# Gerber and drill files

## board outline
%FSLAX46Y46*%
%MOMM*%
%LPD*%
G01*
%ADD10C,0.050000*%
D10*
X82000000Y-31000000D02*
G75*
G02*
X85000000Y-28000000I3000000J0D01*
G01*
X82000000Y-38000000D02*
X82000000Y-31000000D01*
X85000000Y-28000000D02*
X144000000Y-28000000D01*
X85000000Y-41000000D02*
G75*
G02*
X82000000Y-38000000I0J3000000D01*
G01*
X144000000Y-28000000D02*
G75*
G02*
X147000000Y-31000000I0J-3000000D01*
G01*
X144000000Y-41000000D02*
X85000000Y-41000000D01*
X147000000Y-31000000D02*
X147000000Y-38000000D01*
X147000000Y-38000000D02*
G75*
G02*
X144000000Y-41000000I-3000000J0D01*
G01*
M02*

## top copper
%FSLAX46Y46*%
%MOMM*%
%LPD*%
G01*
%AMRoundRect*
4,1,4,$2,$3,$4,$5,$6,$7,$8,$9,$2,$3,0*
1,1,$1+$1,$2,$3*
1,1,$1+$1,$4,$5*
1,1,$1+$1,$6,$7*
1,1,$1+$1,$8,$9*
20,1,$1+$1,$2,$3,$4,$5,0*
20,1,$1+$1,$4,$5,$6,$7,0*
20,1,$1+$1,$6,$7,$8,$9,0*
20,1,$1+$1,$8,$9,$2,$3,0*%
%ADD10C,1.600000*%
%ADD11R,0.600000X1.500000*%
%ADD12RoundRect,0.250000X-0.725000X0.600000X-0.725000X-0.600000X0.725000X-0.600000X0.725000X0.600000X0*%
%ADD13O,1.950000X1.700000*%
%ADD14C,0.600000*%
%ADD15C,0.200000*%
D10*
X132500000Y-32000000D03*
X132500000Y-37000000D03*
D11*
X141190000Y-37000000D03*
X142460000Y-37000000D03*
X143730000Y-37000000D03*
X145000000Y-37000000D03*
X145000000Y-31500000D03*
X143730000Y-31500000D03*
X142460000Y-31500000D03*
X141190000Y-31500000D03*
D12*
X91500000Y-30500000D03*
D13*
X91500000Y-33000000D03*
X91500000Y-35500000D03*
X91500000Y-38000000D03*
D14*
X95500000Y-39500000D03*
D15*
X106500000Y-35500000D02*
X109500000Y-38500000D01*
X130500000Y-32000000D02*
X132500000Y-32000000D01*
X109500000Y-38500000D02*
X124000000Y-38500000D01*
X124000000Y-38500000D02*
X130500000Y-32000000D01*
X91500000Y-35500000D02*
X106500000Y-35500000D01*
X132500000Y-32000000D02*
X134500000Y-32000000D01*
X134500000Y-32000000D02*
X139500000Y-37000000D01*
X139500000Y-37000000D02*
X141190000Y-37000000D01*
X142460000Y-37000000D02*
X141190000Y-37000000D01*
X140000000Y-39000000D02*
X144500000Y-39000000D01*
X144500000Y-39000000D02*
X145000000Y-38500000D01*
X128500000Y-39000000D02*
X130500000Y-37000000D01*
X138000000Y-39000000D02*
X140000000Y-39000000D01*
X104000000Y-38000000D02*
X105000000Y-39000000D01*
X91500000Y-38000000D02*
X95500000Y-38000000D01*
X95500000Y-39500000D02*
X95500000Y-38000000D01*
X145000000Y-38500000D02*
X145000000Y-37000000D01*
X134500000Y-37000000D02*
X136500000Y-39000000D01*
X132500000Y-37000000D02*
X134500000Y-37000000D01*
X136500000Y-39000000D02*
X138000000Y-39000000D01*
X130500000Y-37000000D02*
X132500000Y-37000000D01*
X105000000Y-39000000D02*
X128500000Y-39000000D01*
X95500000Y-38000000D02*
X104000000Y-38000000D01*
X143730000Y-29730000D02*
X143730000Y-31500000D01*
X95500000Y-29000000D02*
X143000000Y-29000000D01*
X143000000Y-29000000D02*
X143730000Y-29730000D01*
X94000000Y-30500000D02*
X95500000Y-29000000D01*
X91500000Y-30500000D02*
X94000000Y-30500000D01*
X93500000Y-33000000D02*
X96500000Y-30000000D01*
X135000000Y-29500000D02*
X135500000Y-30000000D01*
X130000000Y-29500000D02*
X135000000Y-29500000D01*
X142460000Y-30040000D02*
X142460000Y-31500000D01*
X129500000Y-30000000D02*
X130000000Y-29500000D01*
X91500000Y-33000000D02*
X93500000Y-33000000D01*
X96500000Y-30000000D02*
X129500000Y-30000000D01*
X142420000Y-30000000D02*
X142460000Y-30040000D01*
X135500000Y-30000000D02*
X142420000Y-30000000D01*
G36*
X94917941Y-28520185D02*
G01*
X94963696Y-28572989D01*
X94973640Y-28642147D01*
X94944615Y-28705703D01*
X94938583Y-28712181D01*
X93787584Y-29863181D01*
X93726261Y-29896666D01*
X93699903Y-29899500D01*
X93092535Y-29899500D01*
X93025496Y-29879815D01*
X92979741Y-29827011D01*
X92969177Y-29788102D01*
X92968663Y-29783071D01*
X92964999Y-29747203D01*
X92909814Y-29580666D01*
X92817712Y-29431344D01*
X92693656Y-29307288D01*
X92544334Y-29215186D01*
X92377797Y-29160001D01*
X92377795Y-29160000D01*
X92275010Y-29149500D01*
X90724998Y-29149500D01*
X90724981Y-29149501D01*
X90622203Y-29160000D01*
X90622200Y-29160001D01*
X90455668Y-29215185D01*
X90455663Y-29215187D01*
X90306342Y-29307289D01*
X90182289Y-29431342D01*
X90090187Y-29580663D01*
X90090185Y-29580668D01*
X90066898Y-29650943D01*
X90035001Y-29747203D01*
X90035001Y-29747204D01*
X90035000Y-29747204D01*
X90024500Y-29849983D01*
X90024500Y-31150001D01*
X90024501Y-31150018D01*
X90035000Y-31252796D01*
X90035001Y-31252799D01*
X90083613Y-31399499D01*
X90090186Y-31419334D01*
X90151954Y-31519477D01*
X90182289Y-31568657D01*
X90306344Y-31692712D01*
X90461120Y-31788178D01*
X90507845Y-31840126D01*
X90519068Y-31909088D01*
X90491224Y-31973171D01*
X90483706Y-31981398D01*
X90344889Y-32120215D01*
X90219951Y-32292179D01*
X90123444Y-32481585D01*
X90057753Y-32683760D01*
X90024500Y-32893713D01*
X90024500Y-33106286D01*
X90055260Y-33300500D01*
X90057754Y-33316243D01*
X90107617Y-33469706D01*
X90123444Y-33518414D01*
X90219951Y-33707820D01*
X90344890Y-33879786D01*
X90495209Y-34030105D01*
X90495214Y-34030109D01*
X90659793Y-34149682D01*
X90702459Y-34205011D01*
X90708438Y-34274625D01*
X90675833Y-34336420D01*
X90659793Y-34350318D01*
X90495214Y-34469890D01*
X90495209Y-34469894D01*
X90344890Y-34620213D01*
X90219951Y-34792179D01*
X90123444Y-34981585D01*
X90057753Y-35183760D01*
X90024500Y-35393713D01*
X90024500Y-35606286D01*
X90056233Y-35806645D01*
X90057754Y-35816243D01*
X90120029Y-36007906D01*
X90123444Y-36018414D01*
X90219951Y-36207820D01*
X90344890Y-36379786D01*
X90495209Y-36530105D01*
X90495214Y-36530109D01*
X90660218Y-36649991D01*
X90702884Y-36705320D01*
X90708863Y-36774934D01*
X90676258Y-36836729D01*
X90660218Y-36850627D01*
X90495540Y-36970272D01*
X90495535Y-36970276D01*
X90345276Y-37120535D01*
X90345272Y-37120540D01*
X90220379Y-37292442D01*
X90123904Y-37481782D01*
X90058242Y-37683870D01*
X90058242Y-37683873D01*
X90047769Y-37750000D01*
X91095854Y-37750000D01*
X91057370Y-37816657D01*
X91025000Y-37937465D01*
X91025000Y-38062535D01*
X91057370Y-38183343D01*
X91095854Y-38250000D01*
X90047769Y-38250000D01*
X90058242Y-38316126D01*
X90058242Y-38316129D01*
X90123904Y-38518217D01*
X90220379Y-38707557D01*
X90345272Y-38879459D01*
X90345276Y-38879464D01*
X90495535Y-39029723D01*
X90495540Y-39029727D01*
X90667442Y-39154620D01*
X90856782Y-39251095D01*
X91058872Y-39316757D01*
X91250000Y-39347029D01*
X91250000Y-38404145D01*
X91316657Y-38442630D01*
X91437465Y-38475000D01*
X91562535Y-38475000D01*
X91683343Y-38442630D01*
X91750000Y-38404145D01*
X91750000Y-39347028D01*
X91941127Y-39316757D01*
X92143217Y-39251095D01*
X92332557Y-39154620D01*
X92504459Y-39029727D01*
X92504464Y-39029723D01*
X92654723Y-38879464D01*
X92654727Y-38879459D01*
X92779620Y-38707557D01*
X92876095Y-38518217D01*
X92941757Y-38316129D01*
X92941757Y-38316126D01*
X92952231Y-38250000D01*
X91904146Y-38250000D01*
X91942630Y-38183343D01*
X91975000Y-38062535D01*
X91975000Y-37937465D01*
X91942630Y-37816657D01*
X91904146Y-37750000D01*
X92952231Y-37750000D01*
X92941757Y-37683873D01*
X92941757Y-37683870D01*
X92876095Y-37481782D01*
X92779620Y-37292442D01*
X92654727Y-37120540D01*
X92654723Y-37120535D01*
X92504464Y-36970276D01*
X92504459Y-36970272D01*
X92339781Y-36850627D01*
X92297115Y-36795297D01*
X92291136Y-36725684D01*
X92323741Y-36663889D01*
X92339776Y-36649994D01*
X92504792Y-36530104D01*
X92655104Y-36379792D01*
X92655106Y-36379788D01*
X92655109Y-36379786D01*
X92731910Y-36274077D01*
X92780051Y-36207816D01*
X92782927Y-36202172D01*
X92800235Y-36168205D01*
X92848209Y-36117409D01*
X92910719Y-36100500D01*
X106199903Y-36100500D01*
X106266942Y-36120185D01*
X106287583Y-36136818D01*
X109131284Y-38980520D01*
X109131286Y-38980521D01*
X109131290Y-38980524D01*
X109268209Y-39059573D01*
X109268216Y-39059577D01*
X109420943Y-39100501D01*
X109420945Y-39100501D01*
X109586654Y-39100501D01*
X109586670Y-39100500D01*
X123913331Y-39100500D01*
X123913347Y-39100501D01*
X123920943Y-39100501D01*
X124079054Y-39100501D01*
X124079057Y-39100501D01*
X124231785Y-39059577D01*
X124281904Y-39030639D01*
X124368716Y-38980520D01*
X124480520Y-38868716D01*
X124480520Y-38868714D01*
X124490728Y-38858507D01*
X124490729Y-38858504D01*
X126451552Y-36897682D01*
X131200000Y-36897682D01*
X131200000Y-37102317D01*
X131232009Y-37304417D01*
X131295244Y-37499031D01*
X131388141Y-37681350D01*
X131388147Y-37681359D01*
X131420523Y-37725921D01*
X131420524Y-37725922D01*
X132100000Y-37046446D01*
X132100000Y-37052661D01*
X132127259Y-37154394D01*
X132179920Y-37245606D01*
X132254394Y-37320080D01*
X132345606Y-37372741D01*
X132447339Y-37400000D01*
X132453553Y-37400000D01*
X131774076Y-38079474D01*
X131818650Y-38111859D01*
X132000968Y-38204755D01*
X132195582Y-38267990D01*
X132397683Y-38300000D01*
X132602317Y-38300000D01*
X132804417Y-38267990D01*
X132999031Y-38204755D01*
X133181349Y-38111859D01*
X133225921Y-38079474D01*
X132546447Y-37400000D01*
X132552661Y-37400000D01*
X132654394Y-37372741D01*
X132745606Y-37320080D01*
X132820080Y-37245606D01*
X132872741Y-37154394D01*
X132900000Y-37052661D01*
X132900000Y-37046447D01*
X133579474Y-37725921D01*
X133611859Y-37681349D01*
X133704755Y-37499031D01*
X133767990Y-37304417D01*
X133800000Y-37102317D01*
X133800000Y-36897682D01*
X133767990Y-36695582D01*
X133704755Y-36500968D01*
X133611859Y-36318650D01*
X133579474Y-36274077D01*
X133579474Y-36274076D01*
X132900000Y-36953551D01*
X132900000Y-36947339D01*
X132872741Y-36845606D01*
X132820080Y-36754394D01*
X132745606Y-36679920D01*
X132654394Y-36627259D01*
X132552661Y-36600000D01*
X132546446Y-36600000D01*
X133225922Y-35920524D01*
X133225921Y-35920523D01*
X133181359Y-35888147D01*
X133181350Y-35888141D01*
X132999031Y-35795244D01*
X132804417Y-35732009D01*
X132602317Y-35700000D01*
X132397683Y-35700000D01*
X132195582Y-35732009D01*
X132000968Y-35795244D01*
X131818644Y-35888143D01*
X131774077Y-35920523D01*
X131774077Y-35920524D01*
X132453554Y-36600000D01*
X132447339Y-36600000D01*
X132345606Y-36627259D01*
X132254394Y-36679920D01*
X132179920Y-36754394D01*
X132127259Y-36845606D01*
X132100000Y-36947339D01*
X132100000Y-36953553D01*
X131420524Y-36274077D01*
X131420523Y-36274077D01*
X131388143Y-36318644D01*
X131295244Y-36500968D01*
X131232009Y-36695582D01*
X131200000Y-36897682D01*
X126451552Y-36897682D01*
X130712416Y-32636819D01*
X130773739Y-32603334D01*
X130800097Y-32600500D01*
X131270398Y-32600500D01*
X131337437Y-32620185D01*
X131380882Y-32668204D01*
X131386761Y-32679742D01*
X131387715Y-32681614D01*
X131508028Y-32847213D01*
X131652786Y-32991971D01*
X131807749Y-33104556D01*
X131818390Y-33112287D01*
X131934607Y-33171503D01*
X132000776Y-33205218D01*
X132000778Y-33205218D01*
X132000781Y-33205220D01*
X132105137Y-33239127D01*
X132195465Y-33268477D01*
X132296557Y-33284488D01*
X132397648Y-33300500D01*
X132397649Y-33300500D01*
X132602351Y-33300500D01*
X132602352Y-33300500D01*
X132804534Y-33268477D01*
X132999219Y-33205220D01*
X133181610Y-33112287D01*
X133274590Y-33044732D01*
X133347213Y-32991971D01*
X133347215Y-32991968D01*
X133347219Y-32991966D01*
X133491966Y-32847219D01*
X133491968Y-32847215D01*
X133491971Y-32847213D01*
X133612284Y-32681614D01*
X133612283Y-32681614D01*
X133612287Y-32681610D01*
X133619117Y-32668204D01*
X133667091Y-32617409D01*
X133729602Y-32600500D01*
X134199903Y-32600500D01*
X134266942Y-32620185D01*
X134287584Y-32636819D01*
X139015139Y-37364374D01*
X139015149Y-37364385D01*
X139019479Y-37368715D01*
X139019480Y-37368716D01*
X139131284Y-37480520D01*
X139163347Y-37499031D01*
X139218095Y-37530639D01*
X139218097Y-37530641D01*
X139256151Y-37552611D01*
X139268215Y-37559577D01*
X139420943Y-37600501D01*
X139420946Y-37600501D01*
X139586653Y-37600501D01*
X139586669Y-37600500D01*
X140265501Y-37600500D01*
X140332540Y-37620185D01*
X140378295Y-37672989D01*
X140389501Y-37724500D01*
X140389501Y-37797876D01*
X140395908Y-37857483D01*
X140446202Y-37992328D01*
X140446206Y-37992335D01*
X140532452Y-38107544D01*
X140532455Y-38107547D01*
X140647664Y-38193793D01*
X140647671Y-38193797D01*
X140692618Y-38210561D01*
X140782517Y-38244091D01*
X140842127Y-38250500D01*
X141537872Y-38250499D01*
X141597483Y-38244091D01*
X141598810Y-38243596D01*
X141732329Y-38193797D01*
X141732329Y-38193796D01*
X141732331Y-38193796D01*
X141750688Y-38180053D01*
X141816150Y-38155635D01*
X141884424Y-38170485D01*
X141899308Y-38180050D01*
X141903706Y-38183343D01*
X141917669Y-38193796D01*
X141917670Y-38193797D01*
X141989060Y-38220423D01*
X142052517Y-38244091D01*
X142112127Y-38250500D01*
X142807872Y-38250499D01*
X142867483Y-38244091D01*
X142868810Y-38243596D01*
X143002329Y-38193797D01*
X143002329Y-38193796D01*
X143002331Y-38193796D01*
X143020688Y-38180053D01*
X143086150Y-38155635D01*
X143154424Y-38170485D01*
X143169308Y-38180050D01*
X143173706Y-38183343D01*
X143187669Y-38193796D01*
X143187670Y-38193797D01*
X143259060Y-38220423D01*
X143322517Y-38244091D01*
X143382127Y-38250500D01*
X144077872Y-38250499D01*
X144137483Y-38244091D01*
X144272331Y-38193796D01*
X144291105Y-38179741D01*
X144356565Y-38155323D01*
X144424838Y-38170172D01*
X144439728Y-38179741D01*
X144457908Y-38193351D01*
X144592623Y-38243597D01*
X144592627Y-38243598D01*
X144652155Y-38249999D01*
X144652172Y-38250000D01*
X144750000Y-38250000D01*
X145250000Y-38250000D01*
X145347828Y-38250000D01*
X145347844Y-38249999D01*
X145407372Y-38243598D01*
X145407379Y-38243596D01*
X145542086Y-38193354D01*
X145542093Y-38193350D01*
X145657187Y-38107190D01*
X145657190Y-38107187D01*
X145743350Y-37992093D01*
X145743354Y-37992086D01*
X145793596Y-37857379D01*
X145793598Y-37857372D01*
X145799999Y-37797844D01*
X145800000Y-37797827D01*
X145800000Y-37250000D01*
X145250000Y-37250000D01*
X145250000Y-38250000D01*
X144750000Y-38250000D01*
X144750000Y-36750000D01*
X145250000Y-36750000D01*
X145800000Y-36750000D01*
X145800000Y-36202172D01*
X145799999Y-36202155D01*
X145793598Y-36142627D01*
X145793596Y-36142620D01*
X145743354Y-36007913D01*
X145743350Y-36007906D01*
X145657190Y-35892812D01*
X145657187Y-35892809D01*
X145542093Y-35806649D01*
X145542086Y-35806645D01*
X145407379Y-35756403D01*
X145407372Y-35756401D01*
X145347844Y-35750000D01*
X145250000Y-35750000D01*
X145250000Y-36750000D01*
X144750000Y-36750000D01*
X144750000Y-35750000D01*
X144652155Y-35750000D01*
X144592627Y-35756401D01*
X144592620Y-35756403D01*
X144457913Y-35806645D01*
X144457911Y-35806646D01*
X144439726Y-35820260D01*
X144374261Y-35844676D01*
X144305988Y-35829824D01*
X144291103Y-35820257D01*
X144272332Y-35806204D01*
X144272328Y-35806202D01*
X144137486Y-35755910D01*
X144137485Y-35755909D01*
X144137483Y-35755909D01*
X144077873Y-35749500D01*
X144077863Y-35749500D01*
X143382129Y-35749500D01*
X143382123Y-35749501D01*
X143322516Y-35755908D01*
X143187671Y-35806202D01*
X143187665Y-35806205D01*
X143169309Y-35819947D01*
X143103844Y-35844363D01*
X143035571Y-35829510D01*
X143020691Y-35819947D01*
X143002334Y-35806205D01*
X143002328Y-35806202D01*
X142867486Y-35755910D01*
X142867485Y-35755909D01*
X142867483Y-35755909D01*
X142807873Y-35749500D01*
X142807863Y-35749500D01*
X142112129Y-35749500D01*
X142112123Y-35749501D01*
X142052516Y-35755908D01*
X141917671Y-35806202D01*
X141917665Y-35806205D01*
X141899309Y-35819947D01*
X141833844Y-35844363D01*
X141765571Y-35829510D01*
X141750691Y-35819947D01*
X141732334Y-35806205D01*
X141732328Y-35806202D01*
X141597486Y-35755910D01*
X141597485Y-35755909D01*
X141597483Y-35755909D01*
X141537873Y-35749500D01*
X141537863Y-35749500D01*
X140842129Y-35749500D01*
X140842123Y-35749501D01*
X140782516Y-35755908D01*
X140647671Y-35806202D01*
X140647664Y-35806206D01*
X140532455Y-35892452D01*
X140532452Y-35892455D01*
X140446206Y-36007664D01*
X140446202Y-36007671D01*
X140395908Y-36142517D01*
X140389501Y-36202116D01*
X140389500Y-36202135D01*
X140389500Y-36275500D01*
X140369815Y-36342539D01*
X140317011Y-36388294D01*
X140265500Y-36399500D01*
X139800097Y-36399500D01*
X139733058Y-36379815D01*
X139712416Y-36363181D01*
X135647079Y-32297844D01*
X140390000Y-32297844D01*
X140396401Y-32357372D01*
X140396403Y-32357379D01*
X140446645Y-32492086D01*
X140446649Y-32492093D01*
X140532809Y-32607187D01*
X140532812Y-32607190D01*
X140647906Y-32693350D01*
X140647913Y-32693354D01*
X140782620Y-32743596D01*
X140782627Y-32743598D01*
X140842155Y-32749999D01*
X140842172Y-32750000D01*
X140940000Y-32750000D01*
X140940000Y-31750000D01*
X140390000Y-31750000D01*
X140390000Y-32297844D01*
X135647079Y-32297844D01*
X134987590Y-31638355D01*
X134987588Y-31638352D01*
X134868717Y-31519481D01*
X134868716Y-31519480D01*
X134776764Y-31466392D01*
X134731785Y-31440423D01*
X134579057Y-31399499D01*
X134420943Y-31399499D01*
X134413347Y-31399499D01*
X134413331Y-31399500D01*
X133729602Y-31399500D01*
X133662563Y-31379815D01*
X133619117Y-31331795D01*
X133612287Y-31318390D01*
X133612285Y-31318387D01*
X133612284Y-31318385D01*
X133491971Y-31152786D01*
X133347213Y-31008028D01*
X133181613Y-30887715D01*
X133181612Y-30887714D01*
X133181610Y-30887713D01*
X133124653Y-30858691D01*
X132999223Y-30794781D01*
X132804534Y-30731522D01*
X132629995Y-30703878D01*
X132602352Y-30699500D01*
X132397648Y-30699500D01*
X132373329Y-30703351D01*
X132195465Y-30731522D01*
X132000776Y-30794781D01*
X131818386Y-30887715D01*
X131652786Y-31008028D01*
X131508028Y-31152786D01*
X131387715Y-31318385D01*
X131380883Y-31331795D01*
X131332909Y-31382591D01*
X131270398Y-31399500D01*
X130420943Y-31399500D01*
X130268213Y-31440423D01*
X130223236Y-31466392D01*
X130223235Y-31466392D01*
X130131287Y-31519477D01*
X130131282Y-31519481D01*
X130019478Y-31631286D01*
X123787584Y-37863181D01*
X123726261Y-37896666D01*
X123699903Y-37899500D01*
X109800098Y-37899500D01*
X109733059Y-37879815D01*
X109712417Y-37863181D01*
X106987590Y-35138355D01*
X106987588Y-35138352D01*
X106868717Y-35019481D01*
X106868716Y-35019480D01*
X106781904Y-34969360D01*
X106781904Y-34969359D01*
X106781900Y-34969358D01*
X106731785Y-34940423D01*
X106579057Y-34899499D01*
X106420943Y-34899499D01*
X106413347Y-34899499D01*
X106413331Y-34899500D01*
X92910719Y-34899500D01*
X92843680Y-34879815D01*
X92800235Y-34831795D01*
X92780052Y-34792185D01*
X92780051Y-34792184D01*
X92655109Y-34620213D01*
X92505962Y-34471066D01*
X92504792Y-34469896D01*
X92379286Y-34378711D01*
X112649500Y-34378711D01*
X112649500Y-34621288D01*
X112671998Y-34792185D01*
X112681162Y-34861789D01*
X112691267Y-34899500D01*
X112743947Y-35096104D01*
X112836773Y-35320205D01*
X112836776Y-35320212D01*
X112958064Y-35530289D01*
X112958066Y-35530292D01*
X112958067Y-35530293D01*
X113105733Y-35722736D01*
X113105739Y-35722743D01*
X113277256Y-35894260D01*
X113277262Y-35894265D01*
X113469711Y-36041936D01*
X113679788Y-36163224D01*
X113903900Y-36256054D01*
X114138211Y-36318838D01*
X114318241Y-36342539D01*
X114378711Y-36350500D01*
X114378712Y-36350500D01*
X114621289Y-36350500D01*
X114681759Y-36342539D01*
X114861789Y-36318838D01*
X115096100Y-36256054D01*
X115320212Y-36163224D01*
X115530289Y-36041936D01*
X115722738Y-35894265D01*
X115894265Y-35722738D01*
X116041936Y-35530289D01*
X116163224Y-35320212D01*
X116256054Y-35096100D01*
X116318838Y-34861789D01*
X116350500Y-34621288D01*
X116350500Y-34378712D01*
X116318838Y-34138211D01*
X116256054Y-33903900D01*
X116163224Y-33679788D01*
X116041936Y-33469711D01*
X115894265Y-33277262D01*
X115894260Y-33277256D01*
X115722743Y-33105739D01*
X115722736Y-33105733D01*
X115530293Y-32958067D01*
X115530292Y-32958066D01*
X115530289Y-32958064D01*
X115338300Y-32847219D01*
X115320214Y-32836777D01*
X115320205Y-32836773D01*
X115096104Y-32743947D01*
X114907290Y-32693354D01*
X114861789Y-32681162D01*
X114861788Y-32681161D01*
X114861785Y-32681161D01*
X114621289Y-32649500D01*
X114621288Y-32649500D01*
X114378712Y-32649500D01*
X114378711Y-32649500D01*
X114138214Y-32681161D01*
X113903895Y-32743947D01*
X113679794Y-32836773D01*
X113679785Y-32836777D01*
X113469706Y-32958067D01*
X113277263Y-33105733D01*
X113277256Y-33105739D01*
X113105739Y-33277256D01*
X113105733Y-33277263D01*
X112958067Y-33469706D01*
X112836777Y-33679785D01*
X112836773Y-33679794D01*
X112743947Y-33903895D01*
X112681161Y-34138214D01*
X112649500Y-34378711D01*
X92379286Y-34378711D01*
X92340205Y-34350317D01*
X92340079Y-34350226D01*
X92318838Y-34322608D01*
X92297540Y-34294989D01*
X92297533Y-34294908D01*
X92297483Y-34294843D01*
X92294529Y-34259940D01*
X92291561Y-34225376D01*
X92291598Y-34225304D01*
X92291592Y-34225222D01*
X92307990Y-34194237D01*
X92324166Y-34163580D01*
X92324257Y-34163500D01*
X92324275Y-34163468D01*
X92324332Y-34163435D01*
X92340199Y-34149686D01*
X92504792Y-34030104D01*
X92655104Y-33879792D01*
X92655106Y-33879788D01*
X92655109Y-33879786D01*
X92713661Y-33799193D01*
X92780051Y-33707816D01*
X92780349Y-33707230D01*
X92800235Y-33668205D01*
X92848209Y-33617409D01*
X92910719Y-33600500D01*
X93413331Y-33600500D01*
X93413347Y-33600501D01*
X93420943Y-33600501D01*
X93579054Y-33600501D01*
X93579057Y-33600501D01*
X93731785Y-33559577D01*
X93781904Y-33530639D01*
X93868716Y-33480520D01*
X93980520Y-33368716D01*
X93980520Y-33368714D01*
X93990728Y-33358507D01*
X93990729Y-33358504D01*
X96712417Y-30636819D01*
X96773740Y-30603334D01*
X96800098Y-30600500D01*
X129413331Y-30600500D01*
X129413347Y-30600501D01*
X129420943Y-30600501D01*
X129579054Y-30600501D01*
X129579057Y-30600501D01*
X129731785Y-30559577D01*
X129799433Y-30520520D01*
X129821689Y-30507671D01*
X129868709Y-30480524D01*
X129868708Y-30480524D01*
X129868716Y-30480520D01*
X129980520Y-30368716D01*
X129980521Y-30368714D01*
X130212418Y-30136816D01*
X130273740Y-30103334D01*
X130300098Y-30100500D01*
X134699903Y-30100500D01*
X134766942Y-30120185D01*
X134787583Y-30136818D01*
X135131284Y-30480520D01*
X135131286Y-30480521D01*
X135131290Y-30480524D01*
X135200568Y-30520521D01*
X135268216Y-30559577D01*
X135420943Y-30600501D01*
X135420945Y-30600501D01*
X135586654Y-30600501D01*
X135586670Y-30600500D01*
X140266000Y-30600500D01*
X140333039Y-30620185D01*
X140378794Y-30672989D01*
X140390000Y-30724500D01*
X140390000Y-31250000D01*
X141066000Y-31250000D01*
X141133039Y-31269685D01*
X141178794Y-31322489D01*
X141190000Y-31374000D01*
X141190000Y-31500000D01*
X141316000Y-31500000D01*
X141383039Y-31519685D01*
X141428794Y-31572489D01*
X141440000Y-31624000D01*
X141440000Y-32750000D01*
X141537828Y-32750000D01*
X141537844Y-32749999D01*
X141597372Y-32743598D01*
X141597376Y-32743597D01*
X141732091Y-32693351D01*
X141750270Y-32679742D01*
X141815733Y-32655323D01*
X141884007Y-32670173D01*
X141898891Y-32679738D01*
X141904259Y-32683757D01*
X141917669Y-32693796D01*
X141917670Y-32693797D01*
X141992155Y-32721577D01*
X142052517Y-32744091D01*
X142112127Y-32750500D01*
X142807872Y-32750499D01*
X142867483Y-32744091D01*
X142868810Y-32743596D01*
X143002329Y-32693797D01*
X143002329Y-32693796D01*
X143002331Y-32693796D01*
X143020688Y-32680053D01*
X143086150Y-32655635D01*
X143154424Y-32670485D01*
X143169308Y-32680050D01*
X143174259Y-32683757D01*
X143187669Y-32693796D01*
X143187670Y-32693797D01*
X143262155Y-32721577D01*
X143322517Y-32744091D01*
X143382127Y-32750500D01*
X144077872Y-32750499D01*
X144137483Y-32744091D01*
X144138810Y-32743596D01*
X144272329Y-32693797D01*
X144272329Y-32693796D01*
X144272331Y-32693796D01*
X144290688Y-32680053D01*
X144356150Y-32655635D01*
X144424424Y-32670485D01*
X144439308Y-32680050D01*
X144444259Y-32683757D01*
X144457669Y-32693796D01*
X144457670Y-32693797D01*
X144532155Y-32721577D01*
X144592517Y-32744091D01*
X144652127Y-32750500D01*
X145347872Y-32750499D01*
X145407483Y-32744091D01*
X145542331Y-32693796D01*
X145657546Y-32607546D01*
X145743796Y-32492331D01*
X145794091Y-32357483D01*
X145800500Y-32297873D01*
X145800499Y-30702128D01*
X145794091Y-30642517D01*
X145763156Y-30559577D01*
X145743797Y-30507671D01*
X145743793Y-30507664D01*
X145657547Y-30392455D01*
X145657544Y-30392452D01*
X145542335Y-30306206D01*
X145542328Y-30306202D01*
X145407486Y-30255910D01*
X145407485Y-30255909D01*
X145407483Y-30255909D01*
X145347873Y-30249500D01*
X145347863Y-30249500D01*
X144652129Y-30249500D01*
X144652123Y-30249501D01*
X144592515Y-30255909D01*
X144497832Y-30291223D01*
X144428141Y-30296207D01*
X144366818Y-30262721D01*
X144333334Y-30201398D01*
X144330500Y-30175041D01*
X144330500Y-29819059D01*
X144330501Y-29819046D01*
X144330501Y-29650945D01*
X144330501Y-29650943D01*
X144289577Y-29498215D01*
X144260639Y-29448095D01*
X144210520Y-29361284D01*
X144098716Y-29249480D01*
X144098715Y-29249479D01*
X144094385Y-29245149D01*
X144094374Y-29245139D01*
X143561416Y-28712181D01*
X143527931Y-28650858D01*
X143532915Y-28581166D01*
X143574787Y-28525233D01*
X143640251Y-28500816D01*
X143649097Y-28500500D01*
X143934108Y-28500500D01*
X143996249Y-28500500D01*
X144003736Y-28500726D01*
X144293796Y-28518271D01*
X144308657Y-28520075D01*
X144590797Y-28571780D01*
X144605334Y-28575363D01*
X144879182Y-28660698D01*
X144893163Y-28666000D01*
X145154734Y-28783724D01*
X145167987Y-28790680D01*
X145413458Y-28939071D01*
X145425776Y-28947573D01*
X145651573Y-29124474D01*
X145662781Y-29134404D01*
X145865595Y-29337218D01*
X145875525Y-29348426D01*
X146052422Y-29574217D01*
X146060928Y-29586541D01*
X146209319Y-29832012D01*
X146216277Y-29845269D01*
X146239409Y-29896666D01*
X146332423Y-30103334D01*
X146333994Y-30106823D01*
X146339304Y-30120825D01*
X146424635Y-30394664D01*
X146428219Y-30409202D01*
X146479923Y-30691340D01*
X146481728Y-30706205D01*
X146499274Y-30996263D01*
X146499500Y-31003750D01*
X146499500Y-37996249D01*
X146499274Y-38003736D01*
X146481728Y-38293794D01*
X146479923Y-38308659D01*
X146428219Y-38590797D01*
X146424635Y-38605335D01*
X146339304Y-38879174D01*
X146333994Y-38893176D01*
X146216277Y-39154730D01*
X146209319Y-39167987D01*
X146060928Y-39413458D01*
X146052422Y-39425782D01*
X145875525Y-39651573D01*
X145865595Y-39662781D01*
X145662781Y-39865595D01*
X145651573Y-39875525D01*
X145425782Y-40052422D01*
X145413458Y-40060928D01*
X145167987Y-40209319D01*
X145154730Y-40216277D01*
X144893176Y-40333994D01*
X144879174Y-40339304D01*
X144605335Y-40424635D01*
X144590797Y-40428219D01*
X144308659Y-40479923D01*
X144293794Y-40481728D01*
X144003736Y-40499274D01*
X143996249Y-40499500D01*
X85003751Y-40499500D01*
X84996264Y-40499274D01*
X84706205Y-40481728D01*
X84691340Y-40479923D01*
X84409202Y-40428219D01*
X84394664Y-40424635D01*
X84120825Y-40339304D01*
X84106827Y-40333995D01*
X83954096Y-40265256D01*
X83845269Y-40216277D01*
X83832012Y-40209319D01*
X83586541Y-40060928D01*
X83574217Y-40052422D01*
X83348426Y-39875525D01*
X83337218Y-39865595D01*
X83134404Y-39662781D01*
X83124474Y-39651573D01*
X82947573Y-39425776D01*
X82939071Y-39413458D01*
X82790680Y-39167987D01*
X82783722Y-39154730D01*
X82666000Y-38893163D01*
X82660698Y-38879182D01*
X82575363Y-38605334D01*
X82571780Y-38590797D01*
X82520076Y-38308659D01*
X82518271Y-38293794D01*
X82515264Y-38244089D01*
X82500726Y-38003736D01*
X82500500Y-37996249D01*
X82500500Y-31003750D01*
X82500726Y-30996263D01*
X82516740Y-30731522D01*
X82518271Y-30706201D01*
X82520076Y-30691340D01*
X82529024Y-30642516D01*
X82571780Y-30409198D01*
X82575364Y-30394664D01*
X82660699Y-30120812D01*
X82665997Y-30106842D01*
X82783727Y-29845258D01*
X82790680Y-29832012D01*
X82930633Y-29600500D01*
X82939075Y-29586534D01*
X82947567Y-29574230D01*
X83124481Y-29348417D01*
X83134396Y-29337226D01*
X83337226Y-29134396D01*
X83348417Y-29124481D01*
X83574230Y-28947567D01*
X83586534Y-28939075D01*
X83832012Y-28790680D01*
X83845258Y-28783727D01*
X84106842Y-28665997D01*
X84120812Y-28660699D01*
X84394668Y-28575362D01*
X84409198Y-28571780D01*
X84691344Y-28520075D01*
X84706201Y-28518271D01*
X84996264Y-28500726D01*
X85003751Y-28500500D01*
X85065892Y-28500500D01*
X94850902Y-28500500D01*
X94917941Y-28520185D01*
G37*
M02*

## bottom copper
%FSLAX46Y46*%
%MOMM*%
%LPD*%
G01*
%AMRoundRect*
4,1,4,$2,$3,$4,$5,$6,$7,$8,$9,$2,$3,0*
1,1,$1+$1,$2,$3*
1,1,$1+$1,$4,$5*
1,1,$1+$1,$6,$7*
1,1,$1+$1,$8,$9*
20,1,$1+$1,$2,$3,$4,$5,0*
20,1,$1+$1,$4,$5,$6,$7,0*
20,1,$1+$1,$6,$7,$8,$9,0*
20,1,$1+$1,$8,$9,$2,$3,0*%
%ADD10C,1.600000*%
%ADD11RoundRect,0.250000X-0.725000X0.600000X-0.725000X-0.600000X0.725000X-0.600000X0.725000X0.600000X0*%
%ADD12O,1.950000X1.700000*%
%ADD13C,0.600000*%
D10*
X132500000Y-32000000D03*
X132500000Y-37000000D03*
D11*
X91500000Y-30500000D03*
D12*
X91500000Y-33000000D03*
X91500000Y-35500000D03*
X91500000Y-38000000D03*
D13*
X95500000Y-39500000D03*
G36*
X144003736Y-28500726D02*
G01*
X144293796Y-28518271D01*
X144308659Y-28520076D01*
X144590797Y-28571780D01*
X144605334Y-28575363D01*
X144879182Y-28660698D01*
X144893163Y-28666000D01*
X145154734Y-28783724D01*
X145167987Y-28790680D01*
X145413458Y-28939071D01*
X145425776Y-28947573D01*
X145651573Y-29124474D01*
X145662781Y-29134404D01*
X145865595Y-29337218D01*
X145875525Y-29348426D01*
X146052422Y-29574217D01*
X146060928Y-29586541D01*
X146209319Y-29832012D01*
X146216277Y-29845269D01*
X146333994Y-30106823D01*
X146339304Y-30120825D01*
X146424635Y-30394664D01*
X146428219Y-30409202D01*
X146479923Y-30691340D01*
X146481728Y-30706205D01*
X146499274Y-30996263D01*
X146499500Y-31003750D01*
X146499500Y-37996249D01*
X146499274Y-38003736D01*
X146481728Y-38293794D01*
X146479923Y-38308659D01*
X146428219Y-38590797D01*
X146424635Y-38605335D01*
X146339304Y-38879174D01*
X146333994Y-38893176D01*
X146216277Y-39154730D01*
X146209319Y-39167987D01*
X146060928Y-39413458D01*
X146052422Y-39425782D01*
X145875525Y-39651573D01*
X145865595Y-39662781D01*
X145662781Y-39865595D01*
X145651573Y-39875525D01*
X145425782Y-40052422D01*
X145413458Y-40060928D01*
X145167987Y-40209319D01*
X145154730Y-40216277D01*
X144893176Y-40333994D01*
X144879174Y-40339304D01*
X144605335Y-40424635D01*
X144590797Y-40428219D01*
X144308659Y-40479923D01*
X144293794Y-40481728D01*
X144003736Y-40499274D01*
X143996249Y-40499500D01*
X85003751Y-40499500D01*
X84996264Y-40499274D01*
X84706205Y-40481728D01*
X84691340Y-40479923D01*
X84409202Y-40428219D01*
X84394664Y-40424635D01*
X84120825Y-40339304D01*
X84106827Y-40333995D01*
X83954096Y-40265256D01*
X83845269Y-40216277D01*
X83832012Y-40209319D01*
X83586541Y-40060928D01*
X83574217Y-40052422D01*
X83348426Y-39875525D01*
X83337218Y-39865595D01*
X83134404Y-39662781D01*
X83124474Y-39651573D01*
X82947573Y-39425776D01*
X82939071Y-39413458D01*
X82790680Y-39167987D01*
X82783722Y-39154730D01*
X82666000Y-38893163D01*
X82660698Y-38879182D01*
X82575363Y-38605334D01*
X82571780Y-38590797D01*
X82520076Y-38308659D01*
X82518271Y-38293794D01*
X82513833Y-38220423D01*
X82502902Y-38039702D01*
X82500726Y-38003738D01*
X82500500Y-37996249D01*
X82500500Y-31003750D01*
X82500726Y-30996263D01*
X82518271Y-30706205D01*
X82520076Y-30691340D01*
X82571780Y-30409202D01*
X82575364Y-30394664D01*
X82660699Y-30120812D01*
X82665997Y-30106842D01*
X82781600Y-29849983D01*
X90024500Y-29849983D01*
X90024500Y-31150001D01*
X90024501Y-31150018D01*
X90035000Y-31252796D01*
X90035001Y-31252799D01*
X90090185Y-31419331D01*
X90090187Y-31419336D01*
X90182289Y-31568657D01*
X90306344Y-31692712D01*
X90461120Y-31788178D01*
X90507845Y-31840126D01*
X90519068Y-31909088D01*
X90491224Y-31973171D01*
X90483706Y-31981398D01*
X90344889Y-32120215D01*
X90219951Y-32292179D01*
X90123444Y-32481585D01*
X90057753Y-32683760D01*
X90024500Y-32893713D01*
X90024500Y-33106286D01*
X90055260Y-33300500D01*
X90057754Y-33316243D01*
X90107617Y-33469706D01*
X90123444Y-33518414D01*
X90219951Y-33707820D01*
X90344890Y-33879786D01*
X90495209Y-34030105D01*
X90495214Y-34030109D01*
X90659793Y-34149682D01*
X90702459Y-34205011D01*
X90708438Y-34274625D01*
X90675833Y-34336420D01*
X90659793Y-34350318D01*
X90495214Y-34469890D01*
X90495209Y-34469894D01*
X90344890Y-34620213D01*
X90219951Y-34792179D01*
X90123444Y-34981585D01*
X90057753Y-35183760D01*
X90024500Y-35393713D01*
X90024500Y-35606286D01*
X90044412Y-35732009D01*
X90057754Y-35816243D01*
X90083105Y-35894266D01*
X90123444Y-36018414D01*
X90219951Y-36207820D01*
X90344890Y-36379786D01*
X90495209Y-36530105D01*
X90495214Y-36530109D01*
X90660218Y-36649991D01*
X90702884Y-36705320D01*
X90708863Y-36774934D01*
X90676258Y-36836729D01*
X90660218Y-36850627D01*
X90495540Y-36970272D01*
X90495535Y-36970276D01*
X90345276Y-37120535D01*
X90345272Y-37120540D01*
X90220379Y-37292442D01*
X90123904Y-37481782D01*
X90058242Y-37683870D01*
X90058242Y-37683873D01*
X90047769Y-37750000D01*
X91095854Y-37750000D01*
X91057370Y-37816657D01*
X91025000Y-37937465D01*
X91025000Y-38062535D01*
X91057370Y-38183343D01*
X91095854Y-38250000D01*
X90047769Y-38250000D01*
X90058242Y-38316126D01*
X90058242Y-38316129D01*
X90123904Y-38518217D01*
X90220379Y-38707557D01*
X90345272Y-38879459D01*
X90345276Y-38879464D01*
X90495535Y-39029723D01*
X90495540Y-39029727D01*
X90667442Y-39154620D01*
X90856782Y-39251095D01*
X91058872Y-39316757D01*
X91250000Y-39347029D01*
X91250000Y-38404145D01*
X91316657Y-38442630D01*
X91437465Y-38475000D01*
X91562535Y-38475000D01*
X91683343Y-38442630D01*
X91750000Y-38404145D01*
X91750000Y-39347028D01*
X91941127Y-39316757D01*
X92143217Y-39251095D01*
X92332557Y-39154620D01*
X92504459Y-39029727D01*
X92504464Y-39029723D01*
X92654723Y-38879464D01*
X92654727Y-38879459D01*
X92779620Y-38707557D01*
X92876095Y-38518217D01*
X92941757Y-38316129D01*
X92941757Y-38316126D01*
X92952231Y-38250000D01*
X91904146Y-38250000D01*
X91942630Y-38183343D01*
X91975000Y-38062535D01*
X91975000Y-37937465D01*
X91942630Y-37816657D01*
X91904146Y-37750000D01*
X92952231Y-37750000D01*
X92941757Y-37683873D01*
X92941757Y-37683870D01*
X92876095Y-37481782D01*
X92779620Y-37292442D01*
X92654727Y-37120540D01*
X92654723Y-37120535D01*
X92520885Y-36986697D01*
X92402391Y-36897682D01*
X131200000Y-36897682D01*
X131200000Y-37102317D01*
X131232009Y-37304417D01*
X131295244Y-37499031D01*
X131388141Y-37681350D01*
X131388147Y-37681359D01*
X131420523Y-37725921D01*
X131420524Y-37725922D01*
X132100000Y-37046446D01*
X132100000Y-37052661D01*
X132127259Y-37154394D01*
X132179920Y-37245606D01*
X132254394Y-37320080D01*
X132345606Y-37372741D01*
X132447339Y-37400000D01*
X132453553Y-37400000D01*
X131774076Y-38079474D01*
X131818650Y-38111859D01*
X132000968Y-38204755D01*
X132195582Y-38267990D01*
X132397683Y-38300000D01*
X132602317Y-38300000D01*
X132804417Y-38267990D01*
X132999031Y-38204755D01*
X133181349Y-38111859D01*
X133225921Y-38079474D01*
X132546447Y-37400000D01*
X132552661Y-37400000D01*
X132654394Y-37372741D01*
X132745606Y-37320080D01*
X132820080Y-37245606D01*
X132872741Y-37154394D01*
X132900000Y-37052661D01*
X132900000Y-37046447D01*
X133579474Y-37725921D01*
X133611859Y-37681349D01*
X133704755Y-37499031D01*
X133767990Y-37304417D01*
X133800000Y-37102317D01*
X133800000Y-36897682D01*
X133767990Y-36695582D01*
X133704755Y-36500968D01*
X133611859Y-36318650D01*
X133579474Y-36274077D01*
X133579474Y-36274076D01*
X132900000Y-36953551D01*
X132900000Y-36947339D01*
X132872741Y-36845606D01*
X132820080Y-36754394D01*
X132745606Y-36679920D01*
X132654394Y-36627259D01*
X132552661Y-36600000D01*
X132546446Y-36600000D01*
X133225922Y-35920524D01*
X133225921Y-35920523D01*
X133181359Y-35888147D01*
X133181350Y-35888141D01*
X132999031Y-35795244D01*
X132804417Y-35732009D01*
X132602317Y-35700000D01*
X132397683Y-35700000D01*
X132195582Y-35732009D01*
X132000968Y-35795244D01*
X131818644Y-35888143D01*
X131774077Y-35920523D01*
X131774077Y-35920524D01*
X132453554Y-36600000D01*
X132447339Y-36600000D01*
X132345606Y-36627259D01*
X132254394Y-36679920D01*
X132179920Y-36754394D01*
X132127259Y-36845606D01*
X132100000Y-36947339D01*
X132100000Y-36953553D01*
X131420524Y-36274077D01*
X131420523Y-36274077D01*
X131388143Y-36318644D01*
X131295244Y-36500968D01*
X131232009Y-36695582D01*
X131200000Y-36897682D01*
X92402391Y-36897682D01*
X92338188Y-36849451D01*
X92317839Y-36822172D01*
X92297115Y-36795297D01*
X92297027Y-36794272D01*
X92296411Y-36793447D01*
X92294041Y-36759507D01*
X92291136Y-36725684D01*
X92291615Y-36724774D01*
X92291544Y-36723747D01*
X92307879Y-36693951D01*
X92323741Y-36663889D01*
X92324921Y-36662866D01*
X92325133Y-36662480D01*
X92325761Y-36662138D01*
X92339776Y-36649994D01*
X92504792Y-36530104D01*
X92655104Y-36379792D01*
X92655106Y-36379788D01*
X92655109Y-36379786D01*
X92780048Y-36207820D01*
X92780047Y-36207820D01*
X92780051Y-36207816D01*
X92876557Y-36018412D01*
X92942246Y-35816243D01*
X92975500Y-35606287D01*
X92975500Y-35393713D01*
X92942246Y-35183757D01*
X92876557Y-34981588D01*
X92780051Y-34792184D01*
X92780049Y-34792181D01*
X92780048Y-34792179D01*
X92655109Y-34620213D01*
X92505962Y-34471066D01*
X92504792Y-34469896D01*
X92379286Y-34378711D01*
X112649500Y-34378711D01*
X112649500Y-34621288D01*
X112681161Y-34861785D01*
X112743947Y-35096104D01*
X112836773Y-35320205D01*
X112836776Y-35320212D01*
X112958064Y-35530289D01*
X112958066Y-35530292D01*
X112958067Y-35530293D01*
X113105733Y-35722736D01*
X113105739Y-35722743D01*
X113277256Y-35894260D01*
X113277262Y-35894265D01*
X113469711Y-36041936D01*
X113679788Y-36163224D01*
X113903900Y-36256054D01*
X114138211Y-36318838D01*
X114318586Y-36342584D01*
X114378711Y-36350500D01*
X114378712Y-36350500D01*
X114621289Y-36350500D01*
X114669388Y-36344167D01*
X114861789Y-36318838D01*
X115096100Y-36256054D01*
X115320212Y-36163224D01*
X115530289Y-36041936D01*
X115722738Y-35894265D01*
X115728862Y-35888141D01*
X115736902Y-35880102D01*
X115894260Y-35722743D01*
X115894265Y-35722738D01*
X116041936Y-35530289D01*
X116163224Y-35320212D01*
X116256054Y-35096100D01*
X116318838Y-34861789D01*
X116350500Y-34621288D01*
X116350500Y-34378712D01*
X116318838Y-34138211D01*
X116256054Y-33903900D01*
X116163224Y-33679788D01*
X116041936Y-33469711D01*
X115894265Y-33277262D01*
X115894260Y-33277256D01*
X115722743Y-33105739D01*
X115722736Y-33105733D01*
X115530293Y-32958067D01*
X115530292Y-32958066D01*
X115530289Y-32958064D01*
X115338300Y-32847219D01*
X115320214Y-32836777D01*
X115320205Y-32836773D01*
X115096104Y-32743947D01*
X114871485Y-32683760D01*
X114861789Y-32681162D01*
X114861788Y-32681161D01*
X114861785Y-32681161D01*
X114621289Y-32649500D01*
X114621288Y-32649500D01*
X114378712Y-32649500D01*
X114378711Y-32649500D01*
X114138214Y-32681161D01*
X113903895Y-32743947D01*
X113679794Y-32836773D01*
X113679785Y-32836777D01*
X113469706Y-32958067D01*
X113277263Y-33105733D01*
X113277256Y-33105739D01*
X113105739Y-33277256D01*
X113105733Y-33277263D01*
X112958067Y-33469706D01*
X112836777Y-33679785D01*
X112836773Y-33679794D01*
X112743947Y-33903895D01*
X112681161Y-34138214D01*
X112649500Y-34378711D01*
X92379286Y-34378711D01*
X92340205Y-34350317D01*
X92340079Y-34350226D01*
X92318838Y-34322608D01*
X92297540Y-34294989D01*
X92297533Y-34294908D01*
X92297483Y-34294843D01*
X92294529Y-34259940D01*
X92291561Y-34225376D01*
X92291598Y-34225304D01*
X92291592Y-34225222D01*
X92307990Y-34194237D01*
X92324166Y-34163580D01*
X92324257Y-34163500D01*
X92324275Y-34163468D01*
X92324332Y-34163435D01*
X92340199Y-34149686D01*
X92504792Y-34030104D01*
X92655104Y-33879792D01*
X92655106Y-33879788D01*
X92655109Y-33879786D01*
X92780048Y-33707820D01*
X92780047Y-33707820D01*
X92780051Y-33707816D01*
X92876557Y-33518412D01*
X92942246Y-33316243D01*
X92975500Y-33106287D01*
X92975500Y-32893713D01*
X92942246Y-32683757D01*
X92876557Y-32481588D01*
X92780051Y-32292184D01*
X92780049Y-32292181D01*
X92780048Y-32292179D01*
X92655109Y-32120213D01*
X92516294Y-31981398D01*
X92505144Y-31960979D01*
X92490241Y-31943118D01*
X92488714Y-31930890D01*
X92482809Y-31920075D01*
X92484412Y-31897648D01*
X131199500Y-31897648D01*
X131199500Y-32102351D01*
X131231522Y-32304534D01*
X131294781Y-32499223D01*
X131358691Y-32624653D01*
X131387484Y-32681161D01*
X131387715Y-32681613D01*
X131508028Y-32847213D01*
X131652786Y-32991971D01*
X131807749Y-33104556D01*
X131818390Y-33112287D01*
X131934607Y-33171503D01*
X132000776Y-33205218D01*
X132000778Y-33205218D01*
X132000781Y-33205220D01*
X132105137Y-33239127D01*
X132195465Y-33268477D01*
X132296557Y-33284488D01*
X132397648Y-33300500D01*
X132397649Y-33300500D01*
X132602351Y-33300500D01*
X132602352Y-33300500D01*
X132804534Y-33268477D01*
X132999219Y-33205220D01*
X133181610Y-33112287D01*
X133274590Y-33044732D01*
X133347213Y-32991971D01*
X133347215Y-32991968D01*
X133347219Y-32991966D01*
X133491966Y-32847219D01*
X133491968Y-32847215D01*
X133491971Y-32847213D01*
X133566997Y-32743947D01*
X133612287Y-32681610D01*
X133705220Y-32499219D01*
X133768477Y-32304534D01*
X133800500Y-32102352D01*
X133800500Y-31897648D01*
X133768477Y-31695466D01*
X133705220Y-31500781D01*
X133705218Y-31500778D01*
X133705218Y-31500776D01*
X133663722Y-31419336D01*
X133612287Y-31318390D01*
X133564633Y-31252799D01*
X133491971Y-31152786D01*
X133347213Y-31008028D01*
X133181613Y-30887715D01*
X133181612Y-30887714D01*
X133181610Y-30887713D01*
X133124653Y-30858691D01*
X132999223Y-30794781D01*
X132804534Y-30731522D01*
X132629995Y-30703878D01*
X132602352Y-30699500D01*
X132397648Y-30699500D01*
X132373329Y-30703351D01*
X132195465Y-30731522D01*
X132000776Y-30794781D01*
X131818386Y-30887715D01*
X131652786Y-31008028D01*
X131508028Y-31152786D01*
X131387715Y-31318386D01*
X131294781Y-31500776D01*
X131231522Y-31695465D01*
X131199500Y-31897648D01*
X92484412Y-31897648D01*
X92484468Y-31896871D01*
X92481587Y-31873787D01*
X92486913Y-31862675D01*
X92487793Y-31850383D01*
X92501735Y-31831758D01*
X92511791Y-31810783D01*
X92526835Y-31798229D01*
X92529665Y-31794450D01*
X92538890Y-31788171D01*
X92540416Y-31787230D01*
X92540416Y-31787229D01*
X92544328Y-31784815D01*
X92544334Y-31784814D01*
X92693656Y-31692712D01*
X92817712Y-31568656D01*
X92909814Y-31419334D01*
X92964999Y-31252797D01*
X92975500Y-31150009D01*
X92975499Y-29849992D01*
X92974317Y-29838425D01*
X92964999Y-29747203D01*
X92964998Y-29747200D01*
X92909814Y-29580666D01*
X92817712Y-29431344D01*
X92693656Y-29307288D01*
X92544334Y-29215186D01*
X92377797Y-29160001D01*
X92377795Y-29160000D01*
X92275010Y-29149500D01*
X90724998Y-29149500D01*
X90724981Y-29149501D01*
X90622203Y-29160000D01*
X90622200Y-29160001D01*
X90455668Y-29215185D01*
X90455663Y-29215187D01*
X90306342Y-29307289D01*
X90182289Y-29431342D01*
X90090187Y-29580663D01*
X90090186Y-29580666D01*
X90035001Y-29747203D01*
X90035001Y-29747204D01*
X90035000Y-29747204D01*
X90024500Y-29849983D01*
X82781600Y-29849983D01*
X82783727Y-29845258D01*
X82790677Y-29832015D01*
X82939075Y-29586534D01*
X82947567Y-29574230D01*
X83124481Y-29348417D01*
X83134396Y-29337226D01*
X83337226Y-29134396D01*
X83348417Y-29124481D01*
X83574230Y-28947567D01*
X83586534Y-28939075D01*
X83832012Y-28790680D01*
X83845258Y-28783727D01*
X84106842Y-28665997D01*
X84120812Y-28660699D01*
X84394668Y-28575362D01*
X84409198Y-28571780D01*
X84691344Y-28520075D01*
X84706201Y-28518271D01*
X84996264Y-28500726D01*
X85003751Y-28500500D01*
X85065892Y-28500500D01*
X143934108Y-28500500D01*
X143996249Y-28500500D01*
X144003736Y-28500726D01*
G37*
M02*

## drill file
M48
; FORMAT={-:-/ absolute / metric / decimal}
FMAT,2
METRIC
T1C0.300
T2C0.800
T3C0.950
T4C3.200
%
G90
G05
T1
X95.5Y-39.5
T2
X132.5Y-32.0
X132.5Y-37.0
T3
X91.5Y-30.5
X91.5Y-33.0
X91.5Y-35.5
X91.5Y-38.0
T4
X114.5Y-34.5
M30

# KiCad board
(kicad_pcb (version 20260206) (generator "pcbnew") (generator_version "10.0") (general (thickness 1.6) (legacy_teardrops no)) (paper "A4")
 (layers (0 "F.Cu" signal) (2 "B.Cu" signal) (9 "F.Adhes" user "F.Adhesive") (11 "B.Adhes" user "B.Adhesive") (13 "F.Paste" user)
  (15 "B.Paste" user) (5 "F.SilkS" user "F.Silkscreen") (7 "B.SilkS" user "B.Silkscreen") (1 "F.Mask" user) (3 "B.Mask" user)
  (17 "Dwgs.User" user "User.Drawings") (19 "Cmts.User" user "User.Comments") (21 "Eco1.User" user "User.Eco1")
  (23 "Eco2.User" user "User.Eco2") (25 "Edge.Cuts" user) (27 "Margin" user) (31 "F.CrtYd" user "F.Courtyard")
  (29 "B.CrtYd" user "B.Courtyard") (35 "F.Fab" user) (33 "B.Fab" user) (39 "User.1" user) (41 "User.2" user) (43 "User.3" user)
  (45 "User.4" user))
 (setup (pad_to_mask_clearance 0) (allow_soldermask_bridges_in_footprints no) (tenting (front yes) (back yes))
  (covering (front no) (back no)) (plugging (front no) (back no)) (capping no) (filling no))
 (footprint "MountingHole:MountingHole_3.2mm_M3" (layer "F.Cu") (at 114.5 34.5)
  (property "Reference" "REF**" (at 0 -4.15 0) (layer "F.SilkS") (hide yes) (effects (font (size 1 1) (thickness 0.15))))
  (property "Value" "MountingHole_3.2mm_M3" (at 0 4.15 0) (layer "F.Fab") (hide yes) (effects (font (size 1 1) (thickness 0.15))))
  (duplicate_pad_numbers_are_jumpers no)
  (pad "" np_thru_hole circle (at 0 0) (size 3.2 3.2) (drill 3.2) (layers "*.Cu" "*.Mask")))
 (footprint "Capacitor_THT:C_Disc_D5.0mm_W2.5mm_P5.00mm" (layer "F.Cu") (at 132.5 32 -90)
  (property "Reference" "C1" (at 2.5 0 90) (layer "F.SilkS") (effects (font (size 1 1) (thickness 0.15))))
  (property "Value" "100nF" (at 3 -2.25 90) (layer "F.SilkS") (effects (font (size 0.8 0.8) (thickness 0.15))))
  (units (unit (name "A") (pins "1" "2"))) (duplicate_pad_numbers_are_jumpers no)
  (pad "1" thru_hole circle (at 0 0 270) (size 1.6 1.6) (drill 0.8) (layers "*.Cu" "*.Mask") (remove_unused_layers no)
   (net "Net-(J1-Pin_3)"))
  (pad "2" thru_hole circle (at 5 0 270) (size 1.6 1.6) (drill 0.8) (layers "*.Cu" "*.Mask") (remove_unused_layers no)
   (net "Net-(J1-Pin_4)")))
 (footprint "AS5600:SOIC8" (layer "F.Cu") (at 143.095 34.25)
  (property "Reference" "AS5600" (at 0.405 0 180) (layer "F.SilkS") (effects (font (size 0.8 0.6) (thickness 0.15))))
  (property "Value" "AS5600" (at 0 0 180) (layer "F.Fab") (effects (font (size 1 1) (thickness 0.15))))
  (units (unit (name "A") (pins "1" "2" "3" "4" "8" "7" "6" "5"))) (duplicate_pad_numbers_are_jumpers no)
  (pad "1" smd rect (at -1.905 2.75) (size 0.6 1.5) (layers "F.Cu" "F.Mask" "F.Paste") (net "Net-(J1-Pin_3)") (solder_mask_margin 0.102))
  (pad "2" smd rect (at -0.635 2.75) (size 0.6 1.5) (layers "F.Cu" "F.Mask" "F.Paste") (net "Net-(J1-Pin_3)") (solder_mask_margin 0.102))
  (pad "3" smd rect (at 0.635 2.75) (size 0.6 1.5) (layers "F.Cu" "F.Mask" "F.Paste") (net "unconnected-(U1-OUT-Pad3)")
   (solder_mask_margin 0.102))
  (pad "4" smd rect (at 1.905 2.75) (size 0.6 1.5) (layers "F.Cu" "F.Mask" "F.Paste") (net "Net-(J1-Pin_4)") (solder_mask_margin 0.102))
  (pad "5" smd rect (at 1.905 -2.75) (size 0.6 1.5) (layers "F.Cu" "F.Mask" "F.Paste") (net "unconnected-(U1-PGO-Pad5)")
   (solder_mask_margin 0.102))
  (pad "6" smd rect (at 0.635 -2.75) (size 0.6 1.5) (layers "F.Cu" "F.Mask" "F.Paste") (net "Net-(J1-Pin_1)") (solder_mask_margin 0.102))
  (pad "7" smd rect (at -0.635 -2.75) (size 0.6 1.5) (layers "F.Cu" "F.Mask" "F.Paste") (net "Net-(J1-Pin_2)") (solder_mask_margin 0.102))
  (pad "8" smd rect (at -1.905 -2.75) (size 0.6 1.5) (layers "F.Cu" "F.Mask" "F.Paste") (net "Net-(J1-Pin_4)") (solder_mask_margin 0.102)))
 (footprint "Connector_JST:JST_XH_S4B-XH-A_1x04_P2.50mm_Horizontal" (layer "F.Cu") (at 91.5 30.5 -90)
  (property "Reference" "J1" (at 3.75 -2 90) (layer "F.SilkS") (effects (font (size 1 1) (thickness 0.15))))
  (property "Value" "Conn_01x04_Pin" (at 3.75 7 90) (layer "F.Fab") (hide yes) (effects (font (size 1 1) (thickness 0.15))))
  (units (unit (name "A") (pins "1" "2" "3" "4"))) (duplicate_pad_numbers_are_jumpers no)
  (pad "1" thru_hole roundrect (at 0 0 270) (size 1.7 1.95) (drill 0.95) (layers "*.Cu" "*.Mask") (remove_unused_layers no)
   (roundrect_rratio 0.147059) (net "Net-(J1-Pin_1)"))
  (pad "2" thru_hole oval (at 2.5 0 270) (size 1.7 1.95) (drill 0.95) (layers "*.Cu" "*.Mask") (remove_unused_layers no)
   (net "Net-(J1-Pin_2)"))
  (pad "3" thru_hole oval (at 5 0 270) (size 1.7 1.95) (drill 0.95) (layers "*.Cu" "*.Mask") (remove_unused_layers no)
   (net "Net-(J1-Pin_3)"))
  (pad "4" thru_hole oval (at 7.5 0 270) (size 1.7 1.95) (drill 0.95) (layers "*.Cu" "*.Mask") (remove_unused_layers no)
   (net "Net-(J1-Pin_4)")))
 (gr_arc (start 82 31) (mid 82.87868 28.87868) (end 85 28) (stroke (width 0.05) (type default)) (layer "Edge.Cuts"))
 (gr_line (start 82 38) (end 82 31) (stroke (width 0.05) (type default)) (layer "Edge.Cuts"))
 (gr_line (start 85 28) (end 144 28) (stroke (width 0.05) (type default)) (layer "Edge.Cuts"))
 (gr_arc (start 85 41) (mid 82.87868 40.12132) (end 82 38) (stroke (width 0.05) (type default)) (layer "Edge.Cuts"))
 (gr_arc (start 144 28) (mid 146.12132 28.87868) (end 147 31) (stroke (width 0.05) (type default)) (layer "Edge.Cuts"))
 (gr_line (start 144 41) (end 85 41) (stroke (width 0.05) (type default)) (layer "Edge.Cuts"))
 (gr_line (start 147 31) (end 147 38) (stroke (width 0.05) (type default)) (layer "Edge.Cuts"))
 (gr_arc (start 147 38) (mid 146.12132 40.12132) (end 144 41) (stroke (width 0.05) (type default)) (layer "Edge.Cuts"))
 (segment (start 106.5 35.5) (end 109.5 38.5) (width 0.2) (layer "F.Cu") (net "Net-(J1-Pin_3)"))
 (segment (start 130.5 32) (end 132.5 32) (width 0.2) (layer "F.Cu") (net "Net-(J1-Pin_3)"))
 (segment (start 109.5 38.5) (end 124 38.5) (width 0.2) (layer "F.Cu") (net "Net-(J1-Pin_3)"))
 (segment (start 124 38.5) (end 130.5 32) (width 0.2) (layer "F.Cu") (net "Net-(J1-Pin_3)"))
 (segment (start 91.5 35.5) (end 106.5 35.5) (width 0.2) (layer "F.Cu") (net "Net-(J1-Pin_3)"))
 (segment (start 132.5 32) (end 134.5 32) (width 0.2) (layer "F.Cu") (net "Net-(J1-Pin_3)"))
 (segment (start 134.5 32) (end 139.5 37) (width 0.2) (layer "F.Cu") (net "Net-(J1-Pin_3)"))
 (segment (start 139.5 37) (end 141.19 37) (width 0.2) (layer "F.Cu") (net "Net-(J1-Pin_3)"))
 (segment (start 142.46 37) (end 141.19 37) (width 0.2) (layer "F.Cu") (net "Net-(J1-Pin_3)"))
 (segment (start 140 39) (end 144.5 39) (width 0.2) (layer "F.Cu") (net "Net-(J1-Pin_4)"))
 (segment (start 144.5 39) (end 145 38.5) (width 0.2) (layer "F.Cu") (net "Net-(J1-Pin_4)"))
 (segment (start 128.5 39) (end 130.5 37) (width 0.2) (layer "F.Cu") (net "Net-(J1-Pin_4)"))
 (segment (start 138 39) (end 140 39) (width 0.2) (layer "F.Cu") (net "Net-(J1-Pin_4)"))
 (segment (start 104 38) (end 105 39) (width 0.2) (layer "F.Cu") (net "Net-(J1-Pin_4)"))
 (segment (start 91.5 38) (end 95.5 38) (width 0.2) (layer "F.Cu") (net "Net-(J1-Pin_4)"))
 (segment (start 95.5 39.5) (end 95.5 38) (width 0.2) (layer "F.Cu") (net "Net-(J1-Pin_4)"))
 (segment (start 145 38.5) (end 145 37) (width 0.2) (layer "F.Cu") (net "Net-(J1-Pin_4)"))
 (segment (start 134.5 37) (end 136.5 39) (width 0.2) (layer "F.Cu") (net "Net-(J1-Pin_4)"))
 (segment (start 132.5 37) (end 134.5 37) (width 0.2) (layer "F.Cu") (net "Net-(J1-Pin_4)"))
 (segment (start 136.5 39) (end 138 39) (width 0.2) (layer "F.Cu") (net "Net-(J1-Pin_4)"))
 (segment (start 130.5 37) (end 132.5 37) (width 0.2) (layer "F.Cu") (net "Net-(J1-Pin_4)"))
 (segment (start 105 39) (end 128.5 39) (width 0.2) (layer "F.Cu") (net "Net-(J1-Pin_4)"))
 (segment (start 95.5 38) (end 104 38) (width 0.2) (layer "F.Cu") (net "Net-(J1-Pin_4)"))
 (via (at 95.5 39.5) (size 0.6) (drill 0.3) (layers "F.Cu" "B.Cu") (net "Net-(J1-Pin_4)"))
 (segment (start 143.73 29.73) (end 143.73 31.5) (width 0.2) (layer "F.Cu") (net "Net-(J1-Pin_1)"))
 (segment (start 95.5 29) (end 143 29) (width 0.2) (layer "F.Cu") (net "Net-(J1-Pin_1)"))
 (segment (start 143 29) (end 143.73 29.73) (width 0.2) (layer "F.Cu") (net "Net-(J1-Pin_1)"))
 (segment (start 94 30.5) (end 95.5 29) (width 0.2) (layer "F.Cu") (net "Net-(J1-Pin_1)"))
 (segment (start 91.5 30.5) (end 94 30.5) (width 0.2) (layer "F.Cu") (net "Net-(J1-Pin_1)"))
 (segment (start 93.5 33) (end 96.5 30) (width 0.2) (layer "F.Cu") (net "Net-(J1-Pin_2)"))
 (segment (start 135 29.5) (end 135.5 30) (width 0.2) (layer "F.Cu") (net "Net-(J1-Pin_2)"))
 (segment (start 130 29.5) (end 135 29.5) (width 0.2) (layer "F.Cu") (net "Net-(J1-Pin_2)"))
 (segment (start 142.46 30.04) (end 142.46 31.5) (width 0.2) (layer "F.Cu") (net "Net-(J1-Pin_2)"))
 (segment (start 129.5 30) (end 130 29.5) (width 0.2) (layer "F.Cu") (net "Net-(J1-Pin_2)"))
 (segment (start 91.5 33) (end 93.5 33) (width 0.2) (layer "F.Cu") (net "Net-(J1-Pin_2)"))
 (segment (start 96.5 30) (end 129.5 30) (width 0.2) (layer "F.Cu") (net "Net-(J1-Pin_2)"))
 (segment (start 142.42 30) (end 142.46 30.04) (width 0.2) (layer "F.Cu") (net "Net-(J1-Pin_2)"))
 (segment (start 135.5 30) (end 142.42 30) (width 0.2) (layer "F.Cu") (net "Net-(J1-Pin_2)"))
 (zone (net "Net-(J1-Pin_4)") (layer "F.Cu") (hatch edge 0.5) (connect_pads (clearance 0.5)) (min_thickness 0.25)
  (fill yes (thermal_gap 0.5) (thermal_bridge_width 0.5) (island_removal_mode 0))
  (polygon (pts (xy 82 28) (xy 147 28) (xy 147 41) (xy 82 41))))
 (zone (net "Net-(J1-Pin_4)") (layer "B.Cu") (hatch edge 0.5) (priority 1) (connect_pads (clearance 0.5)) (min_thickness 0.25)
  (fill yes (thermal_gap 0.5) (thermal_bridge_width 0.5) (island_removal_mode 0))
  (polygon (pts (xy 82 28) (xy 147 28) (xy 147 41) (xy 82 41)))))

